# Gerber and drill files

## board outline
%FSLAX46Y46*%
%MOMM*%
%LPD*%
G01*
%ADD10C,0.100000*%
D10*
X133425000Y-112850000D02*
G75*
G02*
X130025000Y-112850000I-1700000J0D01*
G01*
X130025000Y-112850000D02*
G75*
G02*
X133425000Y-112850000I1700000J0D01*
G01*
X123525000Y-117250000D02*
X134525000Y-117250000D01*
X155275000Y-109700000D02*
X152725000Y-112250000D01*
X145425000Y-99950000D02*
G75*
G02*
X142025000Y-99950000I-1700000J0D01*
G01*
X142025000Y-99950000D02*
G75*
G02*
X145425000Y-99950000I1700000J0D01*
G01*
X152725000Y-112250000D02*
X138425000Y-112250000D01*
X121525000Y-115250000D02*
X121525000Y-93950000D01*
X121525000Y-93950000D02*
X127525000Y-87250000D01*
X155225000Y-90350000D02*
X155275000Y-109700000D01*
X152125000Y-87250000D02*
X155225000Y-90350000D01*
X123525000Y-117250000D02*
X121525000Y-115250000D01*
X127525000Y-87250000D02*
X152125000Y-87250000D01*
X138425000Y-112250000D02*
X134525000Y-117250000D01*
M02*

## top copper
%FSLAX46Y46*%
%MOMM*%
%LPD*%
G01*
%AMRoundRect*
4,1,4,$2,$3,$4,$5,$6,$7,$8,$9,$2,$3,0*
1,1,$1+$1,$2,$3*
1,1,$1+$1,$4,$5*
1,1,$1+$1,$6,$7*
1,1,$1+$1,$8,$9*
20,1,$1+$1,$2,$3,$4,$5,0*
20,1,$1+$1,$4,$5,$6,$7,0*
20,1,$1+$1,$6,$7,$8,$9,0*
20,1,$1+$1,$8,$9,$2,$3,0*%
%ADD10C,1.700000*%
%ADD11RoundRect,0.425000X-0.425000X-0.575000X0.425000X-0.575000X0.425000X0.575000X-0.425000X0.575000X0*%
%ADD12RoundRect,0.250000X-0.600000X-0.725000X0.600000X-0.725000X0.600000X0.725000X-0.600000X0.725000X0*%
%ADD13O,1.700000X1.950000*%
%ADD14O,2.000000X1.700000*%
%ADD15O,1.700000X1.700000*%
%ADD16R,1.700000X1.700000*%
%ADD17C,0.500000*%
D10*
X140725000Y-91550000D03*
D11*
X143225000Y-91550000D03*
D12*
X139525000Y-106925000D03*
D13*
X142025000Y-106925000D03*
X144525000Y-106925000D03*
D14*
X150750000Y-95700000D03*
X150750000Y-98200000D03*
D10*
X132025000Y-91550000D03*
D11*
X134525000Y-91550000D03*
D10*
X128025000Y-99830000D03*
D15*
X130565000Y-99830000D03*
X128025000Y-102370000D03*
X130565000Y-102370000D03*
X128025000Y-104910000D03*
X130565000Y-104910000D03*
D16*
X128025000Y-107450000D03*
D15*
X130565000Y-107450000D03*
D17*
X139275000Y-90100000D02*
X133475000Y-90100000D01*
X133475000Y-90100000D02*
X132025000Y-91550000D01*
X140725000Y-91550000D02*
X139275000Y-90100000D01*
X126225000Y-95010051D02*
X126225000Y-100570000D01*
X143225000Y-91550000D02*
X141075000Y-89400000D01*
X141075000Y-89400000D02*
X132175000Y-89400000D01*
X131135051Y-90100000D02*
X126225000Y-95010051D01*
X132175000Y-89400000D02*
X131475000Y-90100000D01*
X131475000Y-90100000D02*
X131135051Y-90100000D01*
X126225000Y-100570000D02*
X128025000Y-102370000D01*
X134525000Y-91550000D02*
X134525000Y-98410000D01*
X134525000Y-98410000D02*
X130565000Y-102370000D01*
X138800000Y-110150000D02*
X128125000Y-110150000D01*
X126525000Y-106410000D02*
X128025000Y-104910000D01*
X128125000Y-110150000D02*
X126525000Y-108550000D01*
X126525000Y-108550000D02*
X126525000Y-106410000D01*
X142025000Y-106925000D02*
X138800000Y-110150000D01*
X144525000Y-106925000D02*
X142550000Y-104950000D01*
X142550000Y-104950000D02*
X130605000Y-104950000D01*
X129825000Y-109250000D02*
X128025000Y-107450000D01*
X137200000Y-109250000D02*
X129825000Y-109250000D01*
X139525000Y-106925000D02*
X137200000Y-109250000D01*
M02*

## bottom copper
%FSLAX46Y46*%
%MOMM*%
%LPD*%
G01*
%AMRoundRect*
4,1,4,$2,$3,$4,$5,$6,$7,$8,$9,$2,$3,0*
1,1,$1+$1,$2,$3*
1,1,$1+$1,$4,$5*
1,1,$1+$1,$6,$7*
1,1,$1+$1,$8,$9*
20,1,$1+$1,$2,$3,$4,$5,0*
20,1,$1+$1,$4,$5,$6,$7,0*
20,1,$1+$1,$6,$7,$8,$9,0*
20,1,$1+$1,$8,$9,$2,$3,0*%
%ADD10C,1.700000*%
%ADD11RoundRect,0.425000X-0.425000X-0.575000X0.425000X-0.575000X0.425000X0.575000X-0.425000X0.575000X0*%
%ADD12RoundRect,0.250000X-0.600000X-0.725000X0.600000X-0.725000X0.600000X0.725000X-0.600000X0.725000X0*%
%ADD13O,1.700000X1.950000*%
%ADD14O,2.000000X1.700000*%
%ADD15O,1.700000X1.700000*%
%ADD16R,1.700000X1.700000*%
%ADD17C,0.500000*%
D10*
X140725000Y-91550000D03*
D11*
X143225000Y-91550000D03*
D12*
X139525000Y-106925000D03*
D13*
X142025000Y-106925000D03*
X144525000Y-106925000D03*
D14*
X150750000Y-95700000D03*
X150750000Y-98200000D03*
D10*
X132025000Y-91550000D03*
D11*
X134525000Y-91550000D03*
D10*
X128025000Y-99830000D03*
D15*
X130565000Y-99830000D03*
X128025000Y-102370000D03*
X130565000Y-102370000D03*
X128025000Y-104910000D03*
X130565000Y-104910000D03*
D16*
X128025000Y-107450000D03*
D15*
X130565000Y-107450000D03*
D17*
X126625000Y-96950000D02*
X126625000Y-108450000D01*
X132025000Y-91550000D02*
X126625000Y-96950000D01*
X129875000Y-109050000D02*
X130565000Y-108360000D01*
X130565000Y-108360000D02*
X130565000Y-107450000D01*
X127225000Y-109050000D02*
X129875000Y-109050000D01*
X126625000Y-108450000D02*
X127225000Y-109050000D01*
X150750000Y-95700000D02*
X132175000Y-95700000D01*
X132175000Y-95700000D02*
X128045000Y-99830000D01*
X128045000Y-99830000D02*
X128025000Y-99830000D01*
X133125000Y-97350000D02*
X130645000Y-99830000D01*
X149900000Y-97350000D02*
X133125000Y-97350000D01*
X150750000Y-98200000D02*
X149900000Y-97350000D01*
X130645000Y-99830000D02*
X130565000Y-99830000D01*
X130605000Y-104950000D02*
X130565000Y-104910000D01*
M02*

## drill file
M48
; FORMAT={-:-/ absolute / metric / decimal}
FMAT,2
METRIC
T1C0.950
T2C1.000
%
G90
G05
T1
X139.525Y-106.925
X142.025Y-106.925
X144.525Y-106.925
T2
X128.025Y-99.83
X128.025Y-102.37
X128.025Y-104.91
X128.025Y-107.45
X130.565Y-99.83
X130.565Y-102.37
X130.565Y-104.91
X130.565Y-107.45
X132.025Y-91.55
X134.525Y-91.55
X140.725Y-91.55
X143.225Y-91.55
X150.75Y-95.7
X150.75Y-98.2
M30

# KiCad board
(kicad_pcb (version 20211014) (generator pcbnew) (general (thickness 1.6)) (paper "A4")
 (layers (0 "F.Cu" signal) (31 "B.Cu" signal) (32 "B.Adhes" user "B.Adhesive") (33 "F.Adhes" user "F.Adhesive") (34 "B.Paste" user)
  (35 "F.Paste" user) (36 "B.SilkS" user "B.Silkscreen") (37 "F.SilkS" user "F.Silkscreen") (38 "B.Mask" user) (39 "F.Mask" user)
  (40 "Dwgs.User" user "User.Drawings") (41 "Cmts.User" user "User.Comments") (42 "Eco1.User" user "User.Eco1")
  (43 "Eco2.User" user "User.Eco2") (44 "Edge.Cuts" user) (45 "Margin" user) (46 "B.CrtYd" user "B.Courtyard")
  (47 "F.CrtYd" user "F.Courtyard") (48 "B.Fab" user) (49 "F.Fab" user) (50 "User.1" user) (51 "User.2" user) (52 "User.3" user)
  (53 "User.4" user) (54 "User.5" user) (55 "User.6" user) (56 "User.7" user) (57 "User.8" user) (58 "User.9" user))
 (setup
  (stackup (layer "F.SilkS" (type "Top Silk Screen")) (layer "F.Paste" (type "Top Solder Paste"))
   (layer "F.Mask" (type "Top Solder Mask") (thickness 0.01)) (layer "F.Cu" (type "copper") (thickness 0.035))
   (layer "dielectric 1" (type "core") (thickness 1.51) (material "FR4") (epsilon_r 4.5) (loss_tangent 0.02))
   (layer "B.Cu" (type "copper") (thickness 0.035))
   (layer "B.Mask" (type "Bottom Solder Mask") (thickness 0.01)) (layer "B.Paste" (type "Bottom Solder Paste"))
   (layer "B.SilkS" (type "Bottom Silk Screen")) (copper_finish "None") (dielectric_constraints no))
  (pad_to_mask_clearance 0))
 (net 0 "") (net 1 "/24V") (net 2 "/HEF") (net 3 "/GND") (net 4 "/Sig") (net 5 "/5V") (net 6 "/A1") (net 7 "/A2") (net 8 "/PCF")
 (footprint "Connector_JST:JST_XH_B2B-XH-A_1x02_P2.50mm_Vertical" (layer "F.Cu") (at 140.725 91.55)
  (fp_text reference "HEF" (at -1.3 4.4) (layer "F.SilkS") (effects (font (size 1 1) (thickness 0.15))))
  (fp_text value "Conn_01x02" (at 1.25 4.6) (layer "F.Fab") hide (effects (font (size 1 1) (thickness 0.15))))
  (pad "1" thru_hole circle (at 0 0) (size 1.7 1.7) (drill 1) (layers *.Cu *.Mask) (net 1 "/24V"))
  (pad "2" thru_hole roundrect (at 2.5 0) (size 1.7 2) (drill 1) (layers *.Cu *.Mask) (roundrect_rratio 0.25) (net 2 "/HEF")))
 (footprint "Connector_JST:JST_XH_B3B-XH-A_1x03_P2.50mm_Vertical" (layer "F.Cu") (at 139.525 106.925)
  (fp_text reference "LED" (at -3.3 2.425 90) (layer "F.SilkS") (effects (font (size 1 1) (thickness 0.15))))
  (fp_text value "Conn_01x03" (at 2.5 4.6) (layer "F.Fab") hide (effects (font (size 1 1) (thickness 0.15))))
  (pad "1" thru_hole roundrect (at 0 0) (size 1.7 1.95) (drill 0.95) (layers *.Cu *.Mask) (roundrect_rratio 0.1470588235) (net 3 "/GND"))
  (pad "2" thru_hole oval (at 2.5 0) (size 1.7 1.95) (drill 0.95) (layers *.Cu *.Mask) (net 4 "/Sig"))
  (pad "3" thru_hole oval (at 5 0) (size 1.7 1.95) (drill 0.95) (layers *.Cu *.Mask) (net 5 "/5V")))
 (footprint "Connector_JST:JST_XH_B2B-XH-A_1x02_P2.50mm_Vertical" (layer "F.Cu") (at 150.75 95.7 -90)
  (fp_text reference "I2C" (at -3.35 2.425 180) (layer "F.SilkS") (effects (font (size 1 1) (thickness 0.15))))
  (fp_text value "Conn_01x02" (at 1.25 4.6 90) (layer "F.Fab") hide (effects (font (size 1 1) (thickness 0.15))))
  (pad "1" thru_hole oval (at 0 0 270) (size 1.7 2) (drill 1) (layers *.Cu *.Mask) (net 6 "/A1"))
  (pad "2" thru_hole oval (at 2.5 0 270) (size 1.7 2) (drill 1) (layers *.Cu *.Mask) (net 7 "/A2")))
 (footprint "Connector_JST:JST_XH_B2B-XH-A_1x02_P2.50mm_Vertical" (layer "F.Cu") (at 132.025 91.55)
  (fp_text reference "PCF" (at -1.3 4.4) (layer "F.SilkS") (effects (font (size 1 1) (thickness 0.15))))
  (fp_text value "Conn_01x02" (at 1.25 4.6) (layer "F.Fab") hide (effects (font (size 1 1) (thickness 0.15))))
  (pad "1" thru_hole circle (at 0 0) (size 1.7 1.7) (drill 1) (layers *.Cu *.Mask) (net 1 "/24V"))
  (pad "2" thru_hole roundrect (at 2.5 0) (size 1.7 2) (drill 1) (layers *.Cu *.Mask) (roundrect_rratio 0.25) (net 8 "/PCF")))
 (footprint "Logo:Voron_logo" (layer "F.Cu") (at 137.925 99.85)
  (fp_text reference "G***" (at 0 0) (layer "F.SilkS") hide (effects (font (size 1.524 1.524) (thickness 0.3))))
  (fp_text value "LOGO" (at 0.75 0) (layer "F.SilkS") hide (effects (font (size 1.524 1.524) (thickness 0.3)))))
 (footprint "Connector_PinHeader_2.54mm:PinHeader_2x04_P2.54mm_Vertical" (layer "F.Cu") (at 128.025 99.83)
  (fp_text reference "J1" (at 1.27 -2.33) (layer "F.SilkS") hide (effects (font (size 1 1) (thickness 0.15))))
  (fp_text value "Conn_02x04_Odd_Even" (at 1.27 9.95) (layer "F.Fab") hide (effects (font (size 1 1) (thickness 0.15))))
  (pad "1" thru_hole circle (at 0 0) (size 1.7 1.7) (drill 1) (layers *.Cu *.Mask) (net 6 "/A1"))
  (pad "2" thru_hole oval (at 2.54 0) (size 1.7 1.7) (drill 1) (layers *.Cu *.Mask) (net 7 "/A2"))
  (pad "3" thru_hole oval (at 0 2.54) (size 1.7 1.7) (drill 1) (layers *.Cu *.Mask) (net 2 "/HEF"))
  (pad "4" thru_hole oval (at 2.54 2.54) (size 1.7 1.7) (drill 1) (layers *.Cu *.Mask) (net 8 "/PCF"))
  (pad "5" thru_hole oval (at 0 5.08) (size 1.7 1.7) (drill 1) (layers *.Cu *.Mask) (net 4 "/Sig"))
  (pad "6" thru_hole oval (at 2.54 5.08) (size 1.7 1.7) (drill 1) (layers *.Cu *.Mask) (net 5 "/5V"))
  (pad "7" thru_hole rect (at 0 7.62) (size 1.7 1.7) (drill 1) (layers *.Cu *.Mask) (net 3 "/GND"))
  (pad "8" thru_hole oval (at 2.54 7.62) (size 1.7 1.7) (drill 1) (layers *.Cu *.Mask) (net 1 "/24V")))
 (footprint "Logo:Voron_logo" (layer "B.Cu") (at 137.925 99.85 180)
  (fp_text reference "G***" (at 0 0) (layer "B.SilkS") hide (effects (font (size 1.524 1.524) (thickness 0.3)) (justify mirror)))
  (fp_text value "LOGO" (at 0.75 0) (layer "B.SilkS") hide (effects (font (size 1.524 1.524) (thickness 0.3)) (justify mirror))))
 (gr_circle (center 131.725 112.85) (end 133.425 112.85) (layer "Edge.Cuts") (width 0.1) (fill none))
 (gr_line (start 123.525 117.25) (end 134.525 117.25) (layer "Edge.Cuts") (width 0.1))
 (gr_line (start 155.275 109.7) (end 152.725 112.25) (layer "Edge.Cuts") (width 0.1))
 (gr_circle (center 143.725 99.95) (end 145.425 99.95) (layer "Edge.Cuts") (width 0.1) (fill none))
 (gr_line (start 152.725 112.25) (end 138.425 112.25) (layer "Edge.Cuts") (width 0.1))
 (gr_line (start 121.525 115.25) (end 121.525 93.95) (layer "Edge.Cuts") (width 0.1))
 (gr_line (start 121.525 93.95) (end 127.525 87.25) (layer "Edge.Cuts") (width 0.1))
 (gr_line (start 155.225 90.35) (end 155.275 109.7) (layer "Edge.Cuts") (width 0.1))
 (gr_line (start 152.125 87.25) (end 155.225 90.35) (layer "Edge.Cuts") (width 0.1))
 (gr_line (start 123.525 117.25) (end 121.525 115.25) (layer "Edge.Cuts") (width 0.1))
 (gr_line (start 127.525 87.25) (end 152.125 87.25) (layer "Edge.Cuts") (width 0.1))
 (gr_line (start 138.425 112.25) (end 134.525 117.25) (layer "Edge.Cuts") (width 0.1))
 (segment (start 139.275 90.1) (end 133.475 90.1) (width 0.5) (layer "F.Cu") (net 1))
 (segment (start 133.475 90.1) (end 132.025 91.55) (width 0.5) (layer "F.Cu") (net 1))
 (segment (start 140.725 91.55) (end 139.275 90.1) (width 0.5) (layer "F.Cu") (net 1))
 (segment (start 126.625 96.95) (end 126.625 108.45) (width 0.5) (layer "B.Cu") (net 1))
 (segment (start 132.025 91.55) (end 126.625 96.95) (width 0.5) (layer "B.Cu") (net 1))
 (segment (start 129.875 109.05) (end 130.565 108.36) (width 0.5) (layer "B.Cu") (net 1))
 (segment (start 130.565 108.36) (end 130.565 107.45) (width 0.5) (layer "B.Cu") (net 1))
 (segment (start 127.225 109.05) (end 129.875 109.05) (width 0.5) (layer "B.Cu") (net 1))
 (segment (start 126.625 108.45) (end 127.225 109.05) (width 0.5) (layer "B.Cu") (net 1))
 (segment (start 126.225 95.010051) (end 126.225 100.57) (width 0.5) (layer "F.Cu") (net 2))
 (segment (start 143.225 91.55) (end 141.075 89.4) (width 0.5) (layer "F.Cu") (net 2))
 (segment (start 141.075 89.4) (end 132.175 89.4) (width 0.5) (layer "F.Cu") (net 2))
 (segment (start 131.135051 90.1) (end 126.225 95.010051) (width 0.5) (layer "F.Cu") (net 2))
 (segment (start 132.175 89.4) (end 131.475 90.1) (width 0.5) (layer "F.Cu") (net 2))
 (segment (start 131.475 90.1) (end 131.135051 90.1) (width 0.5) (layer "F.Cu") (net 2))
 (segment (start 126.225 100.57) (end 128.025 102.37) (width 0.5) (layer "F.Cu") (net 2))
 (segment (start 150.75 95.7) (end 132.175 95.7) (width 0.5) (layer "B.Cu") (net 6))
 (segment (start 132.175 95.7) (end 128.045 99.83) (width 0.5) (layer "B.Cu") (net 6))
 (segment (start 128.045 99.83) (end 128.025 99.83) (width 0.5) (layer "B.Cu") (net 6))
 (segment (start 133.125 97.35) (end 130.645 99.83) (width 0.5) (layer "B.Cu") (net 7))
 (segment (start 149.9 97.35) (end 133.125 97.35) (width 0.5) (layer "B.Cu") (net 7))
 (segment (start 150.75 98.2) (end 149.9 97.35) (width 0.5) (layer "B.Cu") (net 7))
 (segment (start 130.645 99.83) (end 130.565 99.83) (width 0.5) (layer "B.Cu") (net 7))
 (segment (start 134.525 91.55) (end 134.525 98.41) (width 0.5) (layer "F.Cu") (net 8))
 (segment (start 134.525 98.41) (end 130.565 102.37) (width 0.5) (layer "F.Cu") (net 8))
 (segment (start 138.8 110.15) (end 128.125 110.15) (width 0.5) (layer "F.Cu") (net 4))
 (segment (start 126.525 106.41) (end 128.025 104.91) (width 0.5) (layer "F.Cu") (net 4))
 (segment (start 128.125 110.15) (end 126.525 108.55) (width 0.5) (layer "F.Cu") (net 4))
 (segment (start 126.525 108.55) (end 126.525 106.41) (width 0.5) (layer "F.Cu") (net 4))
 (segment (start 142.025 106.925) (end 138.8 110.15) (width 0.5) (layer "F.Cu") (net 4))
 (segment (start 144.525 106.925) (end 142.55 104.95) (width 0.5) (layer "F.Cu") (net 5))
 (segment (start 142.55 104.95) (end 130.605 104.95) (width 0.5) (layer "F.Cu") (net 5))
 (segment (start 130.605 104.95) (end 130.565 104.91) (width 0.5) (layer "B.Cu") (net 5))
 (segment (start 129.825 109.25) (end 128.025 107.45) (width 0.5) (layer "F.Cu") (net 3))
 (segment (start 137.2 109.25) (end 129.825 109.25) (width 0.5) (layer "F.Cu") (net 3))
 (segment (start 139.525 106.925) (end 137.2 109.25) (width 0.5) (layer "F.Cu") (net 3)))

